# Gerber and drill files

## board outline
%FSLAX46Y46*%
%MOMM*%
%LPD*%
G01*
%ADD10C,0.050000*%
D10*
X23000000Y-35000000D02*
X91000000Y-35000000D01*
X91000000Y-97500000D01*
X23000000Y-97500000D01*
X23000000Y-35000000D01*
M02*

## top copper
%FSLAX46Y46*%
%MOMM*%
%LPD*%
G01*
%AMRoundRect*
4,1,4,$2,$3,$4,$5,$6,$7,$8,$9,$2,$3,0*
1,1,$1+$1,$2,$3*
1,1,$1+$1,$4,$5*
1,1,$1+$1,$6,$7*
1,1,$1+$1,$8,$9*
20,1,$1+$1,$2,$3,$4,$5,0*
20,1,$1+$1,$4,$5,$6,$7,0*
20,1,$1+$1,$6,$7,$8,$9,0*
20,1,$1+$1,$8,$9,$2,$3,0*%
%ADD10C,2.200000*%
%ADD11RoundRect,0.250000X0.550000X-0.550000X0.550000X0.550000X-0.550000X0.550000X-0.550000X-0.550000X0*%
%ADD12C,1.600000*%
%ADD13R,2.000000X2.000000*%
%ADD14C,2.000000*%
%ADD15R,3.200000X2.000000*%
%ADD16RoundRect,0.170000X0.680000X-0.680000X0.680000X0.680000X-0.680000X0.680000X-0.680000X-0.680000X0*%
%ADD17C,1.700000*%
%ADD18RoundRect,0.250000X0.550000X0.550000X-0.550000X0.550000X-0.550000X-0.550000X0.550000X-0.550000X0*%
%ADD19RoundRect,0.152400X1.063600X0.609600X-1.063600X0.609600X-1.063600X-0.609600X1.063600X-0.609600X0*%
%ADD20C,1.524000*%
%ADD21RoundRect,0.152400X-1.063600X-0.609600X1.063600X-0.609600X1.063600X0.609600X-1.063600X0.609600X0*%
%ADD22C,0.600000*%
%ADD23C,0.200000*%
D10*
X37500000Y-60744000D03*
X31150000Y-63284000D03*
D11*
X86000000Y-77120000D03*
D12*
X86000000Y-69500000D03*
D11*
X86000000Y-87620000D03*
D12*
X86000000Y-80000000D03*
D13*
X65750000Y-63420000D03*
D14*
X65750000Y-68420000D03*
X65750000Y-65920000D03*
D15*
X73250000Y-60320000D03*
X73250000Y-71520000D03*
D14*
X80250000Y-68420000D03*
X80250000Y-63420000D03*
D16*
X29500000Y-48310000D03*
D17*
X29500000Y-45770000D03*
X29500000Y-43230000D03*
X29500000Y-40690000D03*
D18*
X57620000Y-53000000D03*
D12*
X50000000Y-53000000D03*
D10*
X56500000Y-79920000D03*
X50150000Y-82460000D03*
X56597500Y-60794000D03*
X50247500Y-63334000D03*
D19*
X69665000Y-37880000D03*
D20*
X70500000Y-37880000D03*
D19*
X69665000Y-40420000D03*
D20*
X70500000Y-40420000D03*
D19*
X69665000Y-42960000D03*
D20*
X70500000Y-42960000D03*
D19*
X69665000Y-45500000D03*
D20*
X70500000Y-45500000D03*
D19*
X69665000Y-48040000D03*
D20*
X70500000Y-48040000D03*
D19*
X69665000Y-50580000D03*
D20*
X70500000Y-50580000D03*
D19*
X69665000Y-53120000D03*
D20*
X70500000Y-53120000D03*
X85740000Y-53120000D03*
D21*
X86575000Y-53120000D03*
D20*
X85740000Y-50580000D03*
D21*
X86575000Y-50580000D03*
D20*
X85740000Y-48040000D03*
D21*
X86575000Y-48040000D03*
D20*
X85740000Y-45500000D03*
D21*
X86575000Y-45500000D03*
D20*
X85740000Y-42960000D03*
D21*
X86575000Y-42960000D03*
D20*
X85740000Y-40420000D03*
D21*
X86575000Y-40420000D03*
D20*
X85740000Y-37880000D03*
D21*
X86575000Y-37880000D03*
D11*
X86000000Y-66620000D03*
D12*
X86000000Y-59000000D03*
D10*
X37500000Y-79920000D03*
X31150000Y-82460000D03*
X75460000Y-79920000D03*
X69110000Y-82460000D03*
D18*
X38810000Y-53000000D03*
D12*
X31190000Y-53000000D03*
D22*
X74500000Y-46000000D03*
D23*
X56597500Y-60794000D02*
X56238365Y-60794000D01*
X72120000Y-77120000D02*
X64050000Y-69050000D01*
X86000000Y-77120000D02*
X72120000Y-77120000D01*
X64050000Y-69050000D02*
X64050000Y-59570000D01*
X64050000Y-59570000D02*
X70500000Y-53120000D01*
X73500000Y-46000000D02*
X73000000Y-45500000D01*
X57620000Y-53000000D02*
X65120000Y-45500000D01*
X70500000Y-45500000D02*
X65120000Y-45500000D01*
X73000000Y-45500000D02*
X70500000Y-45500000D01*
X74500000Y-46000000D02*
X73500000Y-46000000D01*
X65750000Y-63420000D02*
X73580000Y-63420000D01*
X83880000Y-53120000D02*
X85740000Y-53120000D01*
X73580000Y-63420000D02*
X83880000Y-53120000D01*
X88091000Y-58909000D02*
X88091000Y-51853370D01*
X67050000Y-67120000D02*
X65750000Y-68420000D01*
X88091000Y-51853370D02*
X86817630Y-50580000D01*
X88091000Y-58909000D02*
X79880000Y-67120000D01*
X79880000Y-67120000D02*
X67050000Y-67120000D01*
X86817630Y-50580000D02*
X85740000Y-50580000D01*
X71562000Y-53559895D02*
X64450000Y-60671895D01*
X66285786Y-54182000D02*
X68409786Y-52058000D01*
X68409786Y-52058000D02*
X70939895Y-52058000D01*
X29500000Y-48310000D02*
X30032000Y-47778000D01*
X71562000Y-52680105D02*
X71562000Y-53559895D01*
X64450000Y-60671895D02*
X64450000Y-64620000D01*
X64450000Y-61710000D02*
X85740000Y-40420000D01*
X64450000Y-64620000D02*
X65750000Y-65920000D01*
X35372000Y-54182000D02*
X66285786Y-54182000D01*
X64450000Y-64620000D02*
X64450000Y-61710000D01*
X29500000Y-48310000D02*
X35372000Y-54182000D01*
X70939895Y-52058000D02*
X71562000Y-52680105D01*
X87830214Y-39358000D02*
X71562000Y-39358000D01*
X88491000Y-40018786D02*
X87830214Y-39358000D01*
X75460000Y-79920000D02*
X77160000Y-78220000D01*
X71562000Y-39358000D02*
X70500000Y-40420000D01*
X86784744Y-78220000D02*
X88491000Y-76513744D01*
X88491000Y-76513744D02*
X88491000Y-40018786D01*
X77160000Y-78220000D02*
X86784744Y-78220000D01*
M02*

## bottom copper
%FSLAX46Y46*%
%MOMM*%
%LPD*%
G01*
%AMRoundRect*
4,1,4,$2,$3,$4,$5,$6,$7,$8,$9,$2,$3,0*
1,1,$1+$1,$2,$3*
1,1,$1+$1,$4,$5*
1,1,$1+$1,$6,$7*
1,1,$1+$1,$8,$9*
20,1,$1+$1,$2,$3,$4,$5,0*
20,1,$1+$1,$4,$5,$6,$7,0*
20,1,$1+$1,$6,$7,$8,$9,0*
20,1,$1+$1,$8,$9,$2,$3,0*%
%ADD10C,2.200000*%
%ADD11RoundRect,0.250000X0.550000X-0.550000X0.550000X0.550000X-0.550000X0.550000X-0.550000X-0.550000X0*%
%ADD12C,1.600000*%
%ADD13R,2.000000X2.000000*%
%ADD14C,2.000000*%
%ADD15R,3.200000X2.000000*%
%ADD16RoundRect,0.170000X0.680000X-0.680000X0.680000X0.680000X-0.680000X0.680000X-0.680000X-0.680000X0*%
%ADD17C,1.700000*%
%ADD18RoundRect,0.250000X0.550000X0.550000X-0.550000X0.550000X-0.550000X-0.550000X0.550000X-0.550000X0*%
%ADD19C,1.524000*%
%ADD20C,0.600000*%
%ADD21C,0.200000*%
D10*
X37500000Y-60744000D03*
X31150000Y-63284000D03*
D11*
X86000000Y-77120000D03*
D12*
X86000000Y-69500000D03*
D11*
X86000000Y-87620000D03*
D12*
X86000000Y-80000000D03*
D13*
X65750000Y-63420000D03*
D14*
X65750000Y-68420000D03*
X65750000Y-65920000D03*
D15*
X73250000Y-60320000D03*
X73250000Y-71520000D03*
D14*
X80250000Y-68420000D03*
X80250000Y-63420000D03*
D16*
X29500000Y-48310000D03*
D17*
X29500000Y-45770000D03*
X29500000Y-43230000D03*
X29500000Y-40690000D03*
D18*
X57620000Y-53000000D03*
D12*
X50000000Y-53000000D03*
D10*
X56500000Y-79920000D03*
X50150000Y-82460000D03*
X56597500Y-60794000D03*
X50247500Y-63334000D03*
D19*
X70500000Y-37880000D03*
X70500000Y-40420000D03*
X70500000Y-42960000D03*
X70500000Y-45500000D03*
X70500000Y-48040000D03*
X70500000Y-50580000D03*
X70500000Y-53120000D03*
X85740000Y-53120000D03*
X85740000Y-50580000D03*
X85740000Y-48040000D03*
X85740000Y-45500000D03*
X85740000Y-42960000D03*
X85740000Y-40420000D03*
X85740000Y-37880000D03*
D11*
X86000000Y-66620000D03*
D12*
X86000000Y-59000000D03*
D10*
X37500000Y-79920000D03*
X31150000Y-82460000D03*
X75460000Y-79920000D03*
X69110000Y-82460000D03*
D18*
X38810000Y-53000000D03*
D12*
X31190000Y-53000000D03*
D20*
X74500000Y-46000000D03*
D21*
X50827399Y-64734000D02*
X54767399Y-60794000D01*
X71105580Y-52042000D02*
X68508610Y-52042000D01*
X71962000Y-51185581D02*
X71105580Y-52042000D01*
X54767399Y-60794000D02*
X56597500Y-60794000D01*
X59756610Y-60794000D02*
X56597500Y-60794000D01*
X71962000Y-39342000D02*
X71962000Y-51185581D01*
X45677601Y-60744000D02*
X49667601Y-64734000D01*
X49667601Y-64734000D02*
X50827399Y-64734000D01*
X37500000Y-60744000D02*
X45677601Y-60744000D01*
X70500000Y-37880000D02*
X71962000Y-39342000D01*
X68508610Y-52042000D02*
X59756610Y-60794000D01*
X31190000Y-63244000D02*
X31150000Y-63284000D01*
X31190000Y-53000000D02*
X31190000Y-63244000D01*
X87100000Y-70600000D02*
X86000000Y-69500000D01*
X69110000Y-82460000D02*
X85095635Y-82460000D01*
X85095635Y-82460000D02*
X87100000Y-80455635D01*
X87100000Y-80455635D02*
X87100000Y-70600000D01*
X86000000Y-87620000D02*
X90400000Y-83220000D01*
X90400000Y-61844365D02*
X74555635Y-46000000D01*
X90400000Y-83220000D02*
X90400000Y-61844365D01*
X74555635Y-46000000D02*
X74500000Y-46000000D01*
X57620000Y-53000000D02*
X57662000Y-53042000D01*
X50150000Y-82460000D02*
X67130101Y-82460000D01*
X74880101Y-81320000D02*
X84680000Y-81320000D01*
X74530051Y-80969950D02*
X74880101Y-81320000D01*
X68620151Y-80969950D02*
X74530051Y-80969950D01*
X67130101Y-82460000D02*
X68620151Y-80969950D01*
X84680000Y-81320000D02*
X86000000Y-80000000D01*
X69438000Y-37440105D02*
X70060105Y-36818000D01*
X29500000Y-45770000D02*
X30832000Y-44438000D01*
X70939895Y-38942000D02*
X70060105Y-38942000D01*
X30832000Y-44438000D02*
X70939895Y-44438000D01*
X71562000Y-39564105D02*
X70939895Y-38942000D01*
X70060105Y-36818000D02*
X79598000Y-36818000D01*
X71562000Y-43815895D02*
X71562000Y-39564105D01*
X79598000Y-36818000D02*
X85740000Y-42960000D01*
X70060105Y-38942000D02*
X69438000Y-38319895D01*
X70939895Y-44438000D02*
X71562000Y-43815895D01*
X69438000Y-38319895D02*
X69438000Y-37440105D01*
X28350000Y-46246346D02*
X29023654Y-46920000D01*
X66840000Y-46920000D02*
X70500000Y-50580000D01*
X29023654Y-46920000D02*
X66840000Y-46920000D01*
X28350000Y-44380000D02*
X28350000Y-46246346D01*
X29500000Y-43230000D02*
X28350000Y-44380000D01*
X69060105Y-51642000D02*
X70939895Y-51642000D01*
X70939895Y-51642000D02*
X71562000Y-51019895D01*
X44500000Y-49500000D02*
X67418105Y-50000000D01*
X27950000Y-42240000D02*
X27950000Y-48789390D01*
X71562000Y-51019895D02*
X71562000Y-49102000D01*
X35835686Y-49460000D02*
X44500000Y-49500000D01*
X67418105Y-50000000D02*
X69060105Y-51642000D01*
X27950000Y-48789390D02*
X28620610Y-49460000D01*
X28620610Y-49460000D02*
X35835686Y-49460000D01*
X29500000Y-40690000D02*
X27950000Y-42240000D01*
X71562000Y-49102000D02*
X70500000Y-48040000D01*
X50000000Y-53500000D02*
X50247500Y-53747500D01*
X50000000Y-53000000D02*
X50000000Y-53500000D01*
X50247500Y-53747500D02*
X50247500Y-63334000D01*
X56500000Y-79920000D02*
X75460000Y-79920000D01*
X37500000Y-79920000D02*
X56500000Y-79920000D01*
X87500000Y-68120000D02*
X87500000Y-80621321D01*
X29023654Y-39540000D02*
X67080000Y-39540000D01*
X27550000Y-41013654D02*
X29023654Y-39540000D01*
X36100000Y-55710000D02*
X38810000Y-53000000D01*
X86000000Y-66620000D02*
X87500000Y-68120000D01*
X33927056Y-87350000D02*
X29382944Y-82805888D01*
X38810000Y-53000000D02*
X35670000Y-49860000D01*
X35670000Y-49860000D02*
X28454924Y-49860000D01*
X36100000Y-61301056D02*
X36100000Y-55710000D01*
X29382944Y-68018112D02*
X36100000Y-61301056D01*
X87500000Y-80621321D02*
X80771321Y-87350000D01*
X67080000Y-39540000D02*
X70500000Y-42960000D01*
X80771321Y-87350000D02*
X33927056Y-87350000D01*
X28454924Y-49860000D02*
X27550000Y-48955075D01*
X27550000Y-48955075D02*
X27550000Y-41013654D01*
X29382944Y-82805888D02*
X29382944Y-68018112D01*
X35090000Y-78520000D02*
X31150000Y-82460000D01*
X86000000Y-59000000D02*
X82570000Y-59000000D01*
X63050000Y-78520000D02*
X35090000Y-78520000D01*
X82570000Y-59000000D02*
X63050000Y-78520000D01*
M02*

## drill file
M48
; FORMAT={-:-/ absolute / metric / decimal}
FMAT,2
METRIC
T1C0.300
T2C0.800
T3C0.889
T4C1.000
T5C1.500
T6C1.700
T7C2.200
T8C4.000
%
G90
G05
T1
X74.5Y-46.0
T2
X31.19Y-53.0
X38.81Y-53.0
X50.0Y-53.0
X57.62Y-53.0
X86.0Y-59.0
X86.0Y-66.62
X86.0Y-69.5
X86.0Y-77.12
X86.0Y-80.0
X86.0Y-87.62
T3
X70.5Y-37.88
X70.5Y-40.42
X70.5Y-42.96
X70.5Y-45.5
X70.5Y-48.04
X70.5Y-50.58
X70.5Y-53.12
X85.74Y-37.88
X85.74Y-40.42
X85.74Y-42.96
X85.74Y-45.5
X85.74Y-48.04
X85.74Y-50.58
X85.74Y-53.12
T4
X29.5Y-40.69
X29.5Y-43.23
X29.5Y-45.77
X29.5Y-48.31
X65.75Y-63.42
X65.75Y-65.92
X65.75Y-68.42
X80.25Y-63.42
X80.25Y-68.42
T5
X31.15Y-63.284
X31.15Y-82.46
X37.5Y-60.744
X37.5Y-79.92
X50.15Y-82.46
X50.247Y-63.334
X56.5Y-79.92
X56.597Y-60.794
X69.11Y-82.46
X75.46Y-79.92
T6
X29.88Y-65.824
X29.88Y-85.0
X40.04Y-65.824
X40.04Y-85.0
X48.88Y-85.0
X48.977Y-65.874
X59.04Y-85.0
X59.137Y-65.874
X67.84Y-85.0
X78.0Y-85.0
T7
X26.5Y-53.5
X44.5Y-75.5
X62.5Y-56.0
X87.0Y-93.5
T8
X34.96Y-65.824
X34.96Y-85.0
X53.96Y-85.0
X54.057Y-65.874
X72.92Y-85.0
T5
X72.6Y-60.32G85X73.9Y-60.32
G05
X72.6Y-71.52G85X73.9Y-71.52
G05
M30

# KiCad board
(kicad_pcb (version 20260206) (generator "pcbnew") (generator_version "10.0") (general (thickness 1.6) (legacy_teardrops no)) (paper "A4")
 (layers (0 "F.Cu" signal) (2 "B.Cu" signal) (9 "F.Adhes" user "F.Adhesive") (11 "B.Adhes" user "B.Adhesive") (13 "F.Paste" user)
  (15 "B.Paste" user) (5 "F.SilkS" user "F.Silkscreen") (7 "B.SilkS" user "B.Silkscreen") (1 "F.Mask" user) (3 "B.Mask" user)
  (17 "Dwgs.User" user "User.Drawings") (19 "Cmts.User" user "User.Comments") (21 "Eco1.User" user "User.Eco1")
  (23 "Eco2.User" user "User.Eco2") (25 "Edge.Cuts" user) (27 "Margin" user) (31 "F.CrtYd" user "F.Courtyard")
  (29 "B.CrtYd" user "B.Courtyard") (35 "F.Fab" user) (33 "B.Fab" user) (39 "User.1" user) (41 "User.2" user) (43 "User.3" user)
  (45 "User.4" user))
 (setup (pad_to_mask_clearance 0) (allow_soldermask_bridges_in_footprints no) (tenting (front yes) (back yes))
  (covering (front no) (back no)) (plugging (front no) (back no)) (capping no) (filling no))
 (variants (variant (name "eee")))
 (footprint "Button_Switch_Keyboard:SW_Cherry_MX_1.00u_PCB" (layer "F.Cu") (at 37.5 60.744)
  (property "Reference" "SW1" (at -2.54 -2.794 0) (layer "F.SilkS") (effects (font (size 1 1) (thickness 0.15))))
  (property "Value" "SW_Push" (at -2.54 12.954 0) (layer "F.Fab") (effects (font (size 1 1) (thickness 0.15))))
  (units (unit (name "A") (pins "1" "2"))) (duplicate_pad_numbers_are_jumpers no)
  (pad "" np_thru_hole circle (at -7.62 5.08) (size 1.7 1.7) (drill 1.7) (layers "*.Cu" "*.Mask"))
  (pad "" np_thru_hole circle (at -2.54 5.08) (size 4 4) (drill 4) (layers "*.Cu" "*.Mask"))
  (pad "" np_thru_hole circle (at 2.54 5.08) (size 1.7 1.7) (drill 1.7) (layers "*.Cu" "*.Mask"))
  (pad "1" thru_hole circle (at 0 0) (size 2.2 2.2) (drill 1.5) (layers "*.Cu" "*.Mask") (remove_unused_layers no) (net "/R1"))
  (pad "2" thru_hole circle (at -6.35 2.54) (size 2.2 2.2) (drill 1.5) (layers "*.Cu" "*.Mask") (remove_unused_layers no) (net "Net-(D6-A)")))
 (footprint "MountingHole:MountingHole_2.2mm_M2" (layer "F.Cu") (at 87 93.5)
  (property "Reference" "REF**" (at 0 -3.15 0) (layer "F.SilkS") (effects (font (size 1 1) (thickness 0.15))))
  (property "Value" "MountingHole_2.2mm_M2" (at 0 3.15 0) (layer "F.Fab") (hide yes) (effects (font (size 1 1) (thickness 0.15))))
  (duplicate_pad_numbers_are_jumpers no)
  (pad "" np_thru_hole circle (at 0 0) (size 2.2 2.2) (drill 2.2) (layers "*.Cu" "*.Mask")))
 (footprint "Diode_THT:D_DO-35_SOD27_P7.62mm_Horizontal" (layer "F.Cu") (at 86 77.12 90)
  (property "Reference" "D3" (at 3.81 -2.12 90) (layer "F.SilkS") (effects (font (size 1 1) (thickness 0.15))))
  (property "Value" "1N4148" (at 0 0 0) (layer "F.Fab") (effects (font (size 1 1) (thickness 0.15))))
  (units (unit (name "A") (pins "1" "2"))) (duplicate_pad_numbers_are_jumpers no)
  (pad "1" thru_hole roundrect (at 0 0 90) (size 1.6 1.6) (drill 0.8) (layers "*.Cu" "*.Mask") (remove_unused_layers no)
   (roundrect_rratio 0.15625) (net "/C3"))
  (pad "2" thru_hole circle (at 7.62 0 90) (size 1.6 1.6) (drill 0.8) (layers "*.Cu" "*.Mask") (remove_unused_layers no) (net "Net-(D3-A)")))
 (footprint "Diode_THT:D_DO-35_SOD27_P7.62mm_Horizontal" (layer "F.Cu") (at 86 87.62 90)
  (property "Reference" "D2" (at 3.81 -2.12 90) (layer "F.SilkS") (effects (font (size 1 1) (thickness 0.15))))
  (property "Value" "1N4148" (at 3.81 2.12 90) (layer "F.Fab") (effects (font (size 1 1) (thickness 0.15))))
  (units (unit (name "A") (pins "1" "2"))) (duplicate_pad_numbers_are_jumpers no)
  (pad "1" thru_hole roundrect (at 0 0 90) (size 1.6 1.6) (drill 0.8) (layers "*.Cu" "*.Mask") (remove_unused_layers no)
   (roundrect_rratio 0.15625) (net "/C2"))
  (pad "2" thru_hole circle (at 7.62 0 90) (size 1.6 1.6) (drill 0.8) (layers "*.Cu" "*.Mask") (remove_unused_layers no) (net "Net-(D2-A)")))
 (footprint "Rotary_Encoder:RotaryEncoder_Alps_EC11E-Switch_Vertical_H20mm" (layer "F.Cu") (at 65.75 63.42)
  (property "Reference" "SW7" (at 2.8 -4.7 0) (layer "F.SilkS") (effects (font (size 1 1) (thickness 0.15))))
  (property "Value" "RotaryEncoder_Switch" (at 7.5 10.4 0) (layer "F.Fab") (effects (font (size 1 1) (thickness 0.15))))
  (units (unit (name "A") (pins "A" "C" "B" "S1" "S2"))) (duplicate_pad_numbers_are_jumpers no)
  (pad "A" thru_hole rect (at 0 0) (size 2 2) (drill 1) (layers "*.Cu" "*.Mask") (remove_unused_layers no) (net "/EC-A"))
  (pad "B" thru_hole circle (at 0 5) (size 2 2) (drill 1) (layers "*.Cu" "*.Mask") (remove_unused_layers no) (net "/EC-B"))
  (pad "C" thru_hole circle (at 0 2.5) (size 2 2) (drill 1) (layers "*.Cu" "*.Mask") (remove_unused_layers no) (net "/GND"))
  (pad "MP" thru_hole rect (at 7.5 -3.1) (size 3.2 2) (drill oval 2.8 1.5) (layers "*.Cu" "*.Mask") (remove_unused_layers no))
  (pad "MP" thru_hole rect (at 7.5 8.1) (size 3.2 2) (drill oval 2.8 1.5) (layers "*.Cu" "*.Mask") (remove_unused_layers no))
  (pad "S1" thru_hole circle (at 14.5 5) (size 2 2) (drill 1) (layers "*.Cu" "*.Mask") (remove_unused_layers no)
   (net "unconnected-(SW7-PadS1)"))
  (pad "S2" thru_hole circle (at 14.5 0) (size 2 2) (drill 1) (layers "*.Cu" "*.Mask") (remove_unused_layers no)
   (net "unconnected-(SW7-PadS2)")))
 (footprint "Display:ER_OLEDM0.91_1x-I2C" (layer "F.Cu") (at 29.5 48.31 90)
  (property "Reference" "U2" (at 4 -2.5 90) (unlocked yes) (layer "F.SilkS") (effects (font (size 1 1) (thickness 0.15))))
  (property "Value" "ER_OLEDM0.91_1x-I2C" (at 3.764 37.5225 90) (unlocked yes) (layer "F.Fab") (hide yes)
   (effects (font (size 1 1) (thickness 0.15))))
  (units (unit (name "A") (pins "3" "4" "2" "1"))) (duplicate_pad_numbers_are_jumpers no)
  (pad "1" thru_hole roundrect (at 0 0 90) (size 1.7 1.7) (drill 1) (layers "*.Cu" "*.Mask") (remove_unused_layers no)
   (roundrect_rratio 0.1) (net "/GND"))
  (pad "2" thru_hole circle (at 2.54 0 90) (size 1.7 1.7) (drill 1) (layers "*.Cu" "*.Mask") (remove_unused_layers no) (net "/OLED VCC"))
  (pad "3" thru_hole circle (at 5.08 0 90) (size 1.7 1.7) (drill 1) (layers "*.Cu" "*.Mask") (remove_unused_layers no) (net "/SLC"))
  (pad "4" thru_hole circle (at 7.62 0 90) (size 1.7 1.7) (drill 1) (layers "*.Cu" "*.Mask") (remove_unused_layers no) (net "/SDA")))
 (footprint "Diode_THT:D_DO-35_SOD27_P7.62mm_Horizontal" (layer "F.Cu") (at 57.62 53 180)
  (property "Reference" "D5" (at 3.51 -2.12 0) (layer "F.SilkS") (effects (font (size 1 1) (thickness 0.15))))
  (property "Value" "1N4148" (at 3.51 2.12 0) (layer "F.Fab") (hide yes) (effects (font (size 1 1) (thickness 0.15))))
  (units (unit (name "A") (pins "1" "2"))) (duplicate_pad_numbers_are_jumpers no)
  (pad "1" thru_hole roundrect (at 0 0 180) (size 1.6 1.6) (drill 0.8) (layers "*.Cu" "*.Mask") (remove_unused_layers no)
   (roundrect_rratio 0.15625) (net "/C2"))
  (pad "2" thru_hole circle (at 7.62 0 180) (size 1.6 1.6) (drill 0.8) (layers "*.Cu" "*.Mask") (remove_unused_layers no) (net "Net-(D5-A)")))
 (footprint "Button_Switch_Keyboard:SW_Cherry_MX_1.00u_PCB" (layer "F.Cu") (at 56.5 79.92)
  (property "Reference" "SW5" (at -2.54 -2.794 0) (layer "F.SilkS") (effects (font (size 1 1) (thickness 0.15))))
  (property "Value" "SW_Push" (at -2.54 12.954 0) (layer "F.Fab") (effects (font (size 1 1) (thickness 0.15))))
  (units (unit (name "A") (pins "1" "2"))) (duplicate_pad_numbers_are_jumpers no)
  (pad "" np_thru_hole circle (at -7.62 5.08) (size 1.7 1.7) (drill 1.7) (layers "*.Cu" "*.Mask"))
  (pad "" np_thru_hole circle (at -2.54 5.08) (size 4 4) (drill 4) (layers "*.Cu" "*.Mask"))
  (pad "" np_thru_hole circle (at 2.54 5.08) (size 1.7 1.7) (drill 1.7) (layers "*.Cu" "*.Mask"))
  (pad "1" thru_hole circle (at 0 0) (size 2.2 2.2) (drill 1.5) (layers "*.Cu" "*.Mask") (remove_unused_layers no) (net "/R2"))
  (pad "2" thru_hole circle (at -6.35 2.54) (size 2.2 2.2) (drill 1.5) (layers "*.Cu" "*.Mask") (remove_unused_layers no) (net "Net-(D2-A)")))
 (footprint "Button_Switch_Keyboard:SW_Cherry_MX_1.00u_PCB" (layer "F.Cu") (at 56.5975 60.794)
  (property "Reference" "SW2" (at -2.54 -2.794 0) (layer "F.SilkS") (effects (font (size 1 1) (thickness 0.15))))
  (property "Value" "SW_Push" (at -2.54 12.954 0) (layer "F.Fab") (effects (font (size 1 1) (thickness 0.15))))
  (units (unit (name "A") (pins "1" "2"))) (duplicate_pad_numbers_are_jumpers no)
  (pad "" np_thru_hole circle (at -7.62 5.08) (size 1.7 1.7) (drill 1.7) (layers "*.Cu" "*.Mask"))
  (pad "" np_thru_hole circle (at -2.54 5.08) (size 4 4) (drill 4) (layers "*.Cu" "*.Mask"))
  (pad "" np_thru_hole circle (at 2.54 5.08) (size 1.7 1.7) (drill 1.7) (layers "*.Cu" "*.Mask"))
  (pad "1" thru_hole circle (at 0 0) (size 2.2 2.2) (drill 1.5) (layers "*.Cu" "*.Mask") (remove_unused_layers no) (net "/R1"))
  (pad "2" thru_hole circle (at -6.35 2.54) (size 2.2 2.2) (drill 1.5) (layers "*.Cu" "*.Mask") (remove_unused_layers no) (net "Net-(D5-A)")))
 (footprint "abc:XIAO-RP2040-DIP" (layer "F.Cu") (at 78.12 45.5 90)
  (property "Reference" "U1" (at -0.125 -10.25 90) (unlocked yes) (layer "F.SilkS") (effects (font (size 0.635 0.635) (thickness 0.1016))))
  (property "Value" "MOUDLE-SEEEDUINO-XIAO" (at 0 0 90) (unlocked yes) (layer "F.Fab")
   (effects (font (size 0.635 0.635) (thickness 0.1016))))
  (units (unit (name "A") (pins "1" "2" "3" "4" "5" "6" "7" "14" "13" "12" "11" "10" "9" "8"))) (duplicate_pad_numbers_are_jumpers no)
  (pad "1" smd roundrect (at 7.62 -8.455 180) (size 2.432 1.524) (layers "F.Cu" "F.Mask") (roundrect_rratio 0.1) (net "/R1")
   (thermal_bridge_angle 45))
  (pad "1" thru_hole circle (at 7.62 -7.62 180) (size 1.524 1.524) (drill 0.889) (layers "*.Cu" "*.Mask") (remove_unused_layers no)
   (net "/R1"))
  (pad "2" smd roundrect (at 5.08 -8.455 180) (size 2.432 1.524) (layers "F.Cu" "F.Mask") (roundrect_rratio 0.1) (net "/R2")
   (thermal_bridge_angle 45))
  (pad "2" thru_hole circle (at 5.08 -7.62 180) (size 1.524 1.524) (drill 0.889) (layers "*.Cu" "*.Mask") (remove_unused_layers no)
   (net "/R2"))
  (pad "3" smd roundrect (at 2.54 -8.455 180) (size 2.432 1.524) (layers "F.Cu" "F.Mask") (roundrect_rratio 0.1) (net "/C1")
   (thermal_bridge_angle 45))
  (pad "3" thru_hole circle (at 2.54 -7.62 180) (size 1.524 1.524) (drill 0.889) (layers "*.Cu" "*.Mask") (remove_unused_layers no)
   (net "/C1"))
  (pad "4" smd roundrect (at 0 -8.455 180) (size 2.432 1.524) (layers "F.Cu" "F.Mask") (roundrect_rratio 0.1) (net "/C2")
   (thermal_bridge_angle 45))
  (pad "4" thru_hole circle (at 0 -7.62 180) (size 1.524 1.524) (drill 0.889) (layers "*.Cu" "*.Mask") (remove_unused_layers no) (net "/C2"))
  (pad "5" smd roundrect (at -2.54 -8.455 180) (size 2.432 1.524) (layers "F.Cu" "F.Mask") (roundrect_rratio 0.1) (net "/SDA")
   (thermal_bridge_angle 45))
  (pad "5" thru_hole circle (at -2.54 -7.62 180) (size 1.524 1.524) (drill 0.889) (layers "*.Cu" "*.Mask") (remove_unused_layers no)
   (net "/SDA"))
  (pad "6" smd roundrect (at -5.08 -8.455 180) (size 2.432 1.524) (layers "F.Cu" "F.Mask") (roundrect_rratio 0.1) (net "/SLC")
   (thermal_bridge_angle 45))
  (pad "6" thru_hole circle (at -5.08 -7.62 180) (size 1.524 1.524) (drill 0.889) (layers "*.Cu" "*.Mask") (remove_unused_layers no)
   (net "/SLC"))
  (pad "7" smd roundrect (at -7.62 -8.455 180) (size 2.432 1.524) (layers "F.Cu" "F.Mask") (roundrect_rratio 0.1) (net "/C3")
   (thermal_bridge_angle 45))
  (pad "7" thru_hole circle (at -7.62 -7.62 180) (size 1.524 1.524) (drill 0.889) (layers "*.Cu" "*.Mask") (remove_unused_layers no)
   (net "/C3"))
  (pad "8" thru_hole circle (at -7.62 7.62) (size 1.524 1.524) (drill 0.889) (layers "*.Cu" "*.Mask") (remove_unused_layers no)
   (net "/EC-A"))
  (pad "8" smd roundrect (at -7.62 8.455) (size 2.432 1.524) (layers "F.Cu" "F.Mask") (roundrect_rratio 0.1) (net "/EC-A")
   (thermal_bridge_angle 45))
  (pad "9" thru_hole circle (at -5.08 7.62) (size 1.524 1.524) (drill 0.889) (layers "*.Cu" "*.Mask") (remove_unused_layers no)
   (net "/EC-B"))
  (pad "9" smd roundrect (at -5.08 8.455) (size 2.432 1.524) (layers "F.Cu" "F.Mask") (roundrect_rratio 0.1) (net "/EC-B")
   (thermal_bridge_angle 45))
  (pad "10" thru_hole circle (at -2.54 7.62) (size 1.524 1.524) (drill 0.889) (layers "*.Cu" "*.Mask") (remove_unused_layers no)
   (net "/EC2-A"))
  (pad "10" smd roundrect (at -2.54 8.455) (size 2.432 1.524) (layers "F.Cu" "F.Mask") (roundrect_rratio 0.1) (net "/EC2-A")
   (thermal_bridge_angle 45))
  (pad "11" thru_hole circle (at 0 7.62) (size 1.524 1.524) (drill 0.889) (layers "*.Cu" "*.Mask") (remove_unused_layers no) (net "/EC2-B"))
  (pad "11" smd roundrect (at 0 8.455) (size 2.432 1.524) (layers "F.Cu" "F.Mask") (roundrect_rratio 0.1) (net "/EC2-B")
   (thermal_bridge_angle 45))
  (pad "12" thru_hole circle (at 2.54 7.62) (size 1.524 1.524) (drill 0.889) (layers "*.Cu" "*.Mask") (remove_unused_layers no)
   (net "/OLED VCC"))
  (pad "12" smd roundrect (at 2.54 8.455) (size 2.432 1.524) (layers "F.Cu" "F.Mask") (roundrect_rratio 0.1) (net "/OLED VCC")
   (thermal_bridge_angle 45))
  (pad "13" thru_hole circle (at 5.08 7.62) (size 1.524 1.524) (drill 0.889) (layers "*.Cu" "*.Mask") (remove_unused_layers no) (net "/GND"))
  (pad "13" smd roundrect (at 5.08 8.455) (size 2.432 1.524) (layers "F.Cu" "F.Mask") (roundrect_rratio 0.1) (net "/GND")
   (thermal_bridge_angle 45))
  (pad "14" thru_hole circle (at 7.62 7.62) (size 1.524 1.524) (drill 0.889) (layers "*.Cu" "*.Mask") (remove_unused_layers no)
   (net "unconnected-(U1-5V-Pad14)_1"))
  (pad "14" smd roundrect (at 7.62 8.455) (size 2.432 1.524) (layers "F.Cu" "F.Mask") (roundrect_rratio 0.1)
   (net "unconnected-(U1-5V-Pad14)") (thermal_bridge_angle 45)))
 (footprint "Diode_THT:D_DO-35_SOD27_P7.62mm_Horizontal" (layer "F.Cu") (at 86 66.62 90)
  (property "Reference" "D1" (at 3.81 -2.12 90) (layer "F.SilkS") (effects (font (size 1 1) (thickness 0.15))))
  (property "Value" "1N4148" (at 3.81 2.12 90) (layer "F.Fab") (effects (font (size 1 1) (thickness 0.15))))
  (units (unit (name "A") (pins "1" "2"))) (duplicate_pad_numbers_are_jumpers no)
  (pad "1" thru_hole roundrect (at 0 0 90) (size 1.6 1.6) (drill 0.8) (layers "*.Cu" "*.Mask") (remove_unused_layers no)
   (roundrect_rratio 0.15625) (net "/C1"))
  (pad "2" thru_hole circle (at 7.62 0 90) (size 1.6 1.6) (drill 0.8) (layers "*.Cu" "*.Mask") (remove_unused_layers no) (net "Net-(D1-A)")))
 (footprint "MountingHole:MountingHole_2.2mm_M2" (layer "F.Cu") (at 26.5 53.5)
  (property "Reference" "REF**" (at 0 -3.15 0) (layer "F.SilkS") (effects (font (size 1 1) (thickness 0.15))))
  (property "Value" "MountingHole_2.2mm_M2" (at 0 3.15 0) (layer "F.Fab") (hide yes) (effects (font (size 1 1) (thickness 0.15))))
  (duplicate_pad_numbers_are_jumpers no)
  (pad "" np_thru_hole circle (at 0 0) (size 2.2 2.2) (drill 2.2) (layers "*.Cu" "*.Mask")))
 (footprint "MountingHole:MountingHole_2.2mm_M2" (layer "F.Cu") (at 62.5 56)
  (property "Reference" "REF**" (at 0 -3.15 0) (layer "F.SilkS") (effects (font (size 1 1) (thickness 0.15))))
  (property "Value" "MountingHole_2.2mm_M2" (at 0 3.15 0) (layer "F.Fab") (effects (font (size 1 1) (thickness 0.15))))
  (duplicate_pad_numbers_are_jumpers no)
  (pad "" np_thru_hole circle (at 0 0) (size 2.2 2.2) (drill 2.2) (layers "*.Cu" "*.Mask")))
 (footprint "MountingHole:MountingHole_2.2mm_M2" (layer "F.Cu") (at 44.5 75.5)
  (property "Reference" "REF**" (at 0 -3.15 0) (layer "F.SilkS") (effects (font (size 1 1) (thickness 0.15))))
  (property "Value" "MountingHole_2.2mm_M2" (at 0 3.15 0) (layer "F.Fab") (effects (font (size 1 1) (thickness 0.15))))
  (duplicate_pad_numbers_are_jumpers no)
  (pad "" np_thru_hole circle (at 0 0) (size 2.2 2.2) (drill 2.2) (layers "*.Cu" "*.Mask")))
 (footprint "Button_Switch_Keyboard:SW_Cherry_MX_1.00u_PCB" (layer "F.Cu") (at 37.5 79.92)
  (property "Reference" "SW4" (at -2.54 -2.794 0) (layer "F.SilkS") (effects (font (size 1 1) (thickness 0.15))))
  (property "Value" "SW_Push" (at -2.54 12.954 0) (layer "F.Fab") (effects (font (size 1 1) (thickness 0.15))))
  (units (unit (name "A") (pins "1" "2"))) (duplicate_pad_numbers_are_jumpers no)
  (pad "" np_thru_hole circle (at -7.62 5.08) (size 1.7 1.7) (drill 1.7) (layers "*.Cu" "*.Mask"))
  (pad "" np_thru_hole circle (at -2.54 5.08) (size 4 4) (drill 4) (layers "*.Cu" "*.Mask"))
  (pad "" np_thru_hole circle (at 2.54 5.08) (size 1.7 1.7) (drill 1.7) (layers "*.Cu" "*.Mask"))
  (pad "1" thru_hole circle (at 0 0) (size 2.2 2.2) (drill 1.5) (layers "*.Cu" "*.Mask") (remove_unused_layers no) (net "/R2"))
  (pad "2" thru_hole circle (at -6.35 2.54) (size 2.2 2.2) (drill 1.5) (layers "*.Cu" "*.Mask") (remove_unused_layers no) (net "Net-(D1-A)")))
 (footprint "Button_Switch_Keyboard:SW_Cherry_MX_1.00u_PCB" (layer "F.Cu") (at 75.46 79.92)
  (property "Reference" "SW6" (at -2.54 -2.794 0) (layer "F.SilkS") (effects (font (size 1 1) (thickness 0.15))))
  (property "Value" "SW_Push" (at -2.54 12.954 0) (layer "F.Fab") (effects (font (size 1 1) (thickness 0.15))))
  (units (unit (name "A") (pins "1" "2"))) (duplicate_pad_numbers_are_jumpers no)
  (pad "" np_thru_hole circle (at -7.62 5.08) (size 1.7 1.7) (drill 1.7) (layers "*.Cu" "*.Mask"))
  (pad "" np_thru_hole circle (at -2.54 5.08) (size 4 4) (drill 4) (layers "*.Cu" "*.Mask"))
  (pad "" np_thru_hole circle (at 2.54 5.08) (size 1.7 1.7) (drill 1.7) (layers "*.Cu" "*.Mask"))
  (pad "1" thru_hole circle (at 0 0) (size 2.2 2.2) (drill 1.5) (layers "*.Cu" "*.Mask") (remove_unused_layers no) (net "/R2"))
  (pad "2" thru_hole circle (at -6.35 2.54) (size 2.2 2.2) (drill 1.5) (layers "*.Cu" "*.Mask") (remove_unused_layers no) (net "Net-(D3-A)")))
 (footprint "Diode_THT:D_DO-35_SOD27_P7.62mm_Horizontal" (layer "F.Cu") (at 38.81 53 180)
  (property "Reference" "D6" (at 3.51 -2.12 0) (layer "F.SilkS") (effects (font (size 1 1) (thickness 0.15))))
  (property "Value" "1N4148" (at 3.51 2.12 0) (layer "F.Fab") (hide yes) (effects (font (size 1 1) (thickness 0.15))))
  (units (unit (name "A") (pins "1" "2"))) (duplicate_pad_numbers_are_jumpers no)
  (pad "1" thru_hole roundrect (at 0 0 180) (size 1.6 1.6) (drill 0.8) (layers "*.Cu" "*.Mask") (remove_unused_layers no)
   (roundrect_rratio 0.15625) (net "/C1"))
  (pad "2" thru_hole circle (at 7.62 0 180) (size 1.6 1.6) (drill 0.8) (layers "*.Cu" "*.Mask") (remove_unused_layers no) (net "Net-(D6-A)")))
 (gr_rect (start 23 35) (end 91 97.5) (stroke (width 0.05) (type default)) (fill no) (layer "Edge.Cuts"))
 (segment (start 56.5975 60.794) (end 56.238365 60.794) (width 0.2) (layer "F.Cu") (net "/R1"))
 (segment (start 50.827399 64.734) (end 54.767399 60.794) (width 0.2) (layer "B.Cu") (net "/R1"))
 (segment (start 71.10558 52.042) (end 68.50861 52.042) (width 0.2) (layer "B.Cu") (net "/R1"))
 (segment (start 71.962 51.185581) (end 71.10558 52.042) (width 0.2) (layer "B.Cu") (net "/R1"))
 (segment (start 54.767399 60.794) (end 56.5975 60.794) (width 0.2) (layer "B.Cu") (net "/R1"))
 (segment (start 59.75661 60.794) (end 56.5975 60.794) (width 0.2) (layer "B.Cu") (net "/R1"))
 (segment (start 71.962 39.342) (end 71.962 51.185581) (width 0.2) (layer "B.Cu") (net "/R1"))
 (segment (start 45.677601 60.744) (end 49.667601 64.734) (width 0.2) (layer "B.Cu") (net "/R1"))
 (segment (start 49.667601 64.734) (end 50.827399 64.734) (width 0.2) (layer "B.Cu") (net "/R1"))
 (segment (start 37.5 60.744) (end 45.677601 60.744) (width 0.2) (layer "B.Cu") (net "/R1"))
 (segment (start 70.5 37.88) (end 71.962 39.342) (width 0.2) (layer "B.Cu") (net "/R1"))
 (segment (start 68.50861 52.042) (end 59.75661 60.794) (width 0.2) (layer "B.Cu") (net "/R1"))
 (segment (start 31.19 63.244) (end 31.15 63.284) (width 0.2) (layer "B.Cu") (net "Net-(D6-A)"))
 (segment (start 31.19 53) (end 31.19 63.244) (width 0.2) (layer "B.Cu") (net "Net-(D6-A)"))
 (segment (start 72.12 77.12) (end 64.05 69.05) (width 0.2) (layer "F.Cu") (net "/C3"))
 (segment (start 86 77.12) (end 72.12 77.12) (width 0.2) (layer "F.Cu") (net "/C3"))
 (segment (start 64.05 69.05) (end 64.05 59.57) (width 0.2) (layer "F.Cu") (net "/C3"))
 (segment (start 64.05 59.57) (end 70.5 53.12) (width 0.2) (layer "F.Cu") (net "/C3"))
 (segment (start 87.1 70.6) (end 86 69.5) (width 0.2) (layer "B.Cu") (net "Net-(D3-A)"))
 (segment (start 69.11 82.46) (end 85.095635 82.46) (width 0.2) (layer "B.Cu") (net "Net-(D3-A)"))
 (segment (start 85.095635 82.46) (end 87.1 80.455635) (width 0.2) (layer "B.Cu") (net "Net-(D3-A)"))
 (segment (start 87.1 80.455635) (end 87.1 70.6) (width 0.2) (layer "B.Cu") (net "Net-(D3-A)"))
 (segment (start 73.5 46) (end 73 45.5) (width 0.2) (layer "F.Cu") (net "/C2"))
 (segment (start 57.62 53) (end 65.12 45.5) (width 0.2) (layer "F.Cu") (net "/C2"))
 (segment (start 70.5 45.5) (end 65.12 45.5) (width 0.2) (layer "F.Cu") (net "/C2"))
 (segment (start 73 45.5) (end 70.5 45.5) (width 0.2) (layer "F.Cu") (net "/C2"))
 (segment (start 74.5 46) (end 73.5 46) (width 0.2) (layer "F.Cu") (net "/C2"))
 (via (at 74.5 46) (size 0.6) (drill 0.3) (layers "F.Cu" "B.Cu") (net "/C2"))
 (segment (start 86 87.62) (end 90.4 83.22) (width 0.2) (layer "B.Cu") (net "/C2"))
 (segment (start 90.4 61.844365) (end 74.555635 46) (width 0.2) (layer "B.Cu") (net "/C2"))
 (segment (start 90.4 83.22) (end 90.4 61.844365) (width 0.2) (layer "B.Cu") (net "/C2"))
 (segment (start 74.555635 46) (end 74.5 46) (width 0.2) (layer "B.Cu") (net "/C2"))
 (segment (start 57.62 53) (end 57.662 53.042) (width 0.2) (layer "B.Cu") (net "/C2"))
 (segment (start 50.15 82.46) (end 67.130101 82.46) (width 0.2) (layer "B.Cu") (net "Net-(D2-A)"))
 (segment (start 74.880101 81.32) (end 84.68 81.32) (width 0.2) (layer "B.Cu") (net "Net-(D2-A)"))
 (segment (start 74.530051 80.96995) (end 74.880101 81.32) (width 0.2) (layer "B.Cu") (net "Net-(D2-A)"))
 (segment (start 68.620151 80.96995) (end 74.530051 80.96995) (width 0.2) (layer "B.Cu") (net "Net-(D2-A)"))
 (segment (start 67.130101 82.46) (end 68.620151 80.96995) (width 0.2) (layer "B.Cu") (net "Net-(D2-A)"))
 (segment (start 84.68 81.32) (end 86 80) (width 0.2) (layer "B.Cu") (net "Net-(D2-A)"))
 (segment (start 65.75 63.42) (end 73.58 63.42) (width 0.2) (layer "F.Cu") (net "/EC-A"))
 (segment (start 83.88 53.12) (end 85.74 53.12) (width 0.2) (layer "F.Cu") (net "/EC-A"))
 (segment (start 73.58 63.42) (end 83.88 53.12) (width 0.2) (layer "F.Cu") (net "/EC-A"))
 (segment (start 88.091 58.909) (end 88.091 51.85337) (width 0.2) (layer "F.Cu") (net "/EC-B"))
 (segment (start 67.05 67.12) (end 65.75 68.42) (width 0.2) (layer "F.Cu") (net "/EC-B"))
 (segment (start 88.091 51.85337) (end 86.81763 50.58) (width 0.2) (layer "F.Cu") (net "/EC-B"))
 (segment (start 88.091 58.909) (end 79.88 67.12) (width 0.2) (layer "F.Cu") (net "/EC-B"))
 (segment (start 79.88 67.12) (end 67.05 67.12) (width 0.2) (layer "F.Cu") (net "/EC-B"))
 (segment (start 86.81763 50.58) (end 85.74 50.58) (width 0.2) (layer "F.Cu") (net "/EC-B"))
 (segment (start 71.562 53.559895) (end 64.45 60.671895) (width 0.2) (layer "F.Cu") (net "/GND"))
 (segment (start 66.285786 54.182) (end 68.409786 52.058) (width 0.2) (layer "F.Cu") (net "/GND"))
 (segment (start 68.409786 52.058) (end 70.939895 52.058) (width 0.2) (layer "F.Cu") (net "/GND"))
 (segment (start 29.5 48.31) (end 30.032 47.778) (width 0.2) (layer "F.Cu") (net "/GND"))
 (segment (start 71.562 52.680105) (end 71.562 53.559895) (width 0.2) (layer "F.Cu") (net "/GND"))
 (segment (start 64.45 60.671895) (end 64.45 64.62) (width 0.2) (layer "F.Cu") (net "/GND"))
 (segment (start 64.45 61.71) (end 85.74 40.42) (width 0.2) (layer "F.Cu") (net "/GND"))
 (segment (start 64.45 64.62) (end 65.75 65.92) (width 0.2) (layer "F.Cu") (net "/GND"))
 (segment (start 35.372 54.182) (end 66.285786 54.182) (width 0.2) (layer "F.Cu") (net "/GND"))
 (segment (start 64.45 64.62) (end 64.45 61.71) (width 0.2) (layer "F.Cu") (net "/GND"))
 (segment (start 29.5 48.31) (end 35.372 54.182) (width 0.2) (layer "F.Cu") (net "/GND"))
 (segment (start 70.939895 52.058) (end 71.562 52.680105) (width 0.2) (layer "F.Cu") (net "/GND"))
 (segment (start 69.438 37.440105) (end 70.060105 36.818) (width 0.2) (layer "B.Cu") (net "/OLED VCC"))
 (segment (start 29.5 45.77) (end 30.832 44.438) (width 0.2) (layer "B.Cu") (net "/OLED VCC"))
 (segment (start 70.939895 38.942) (end 70.060105 38.942) (width 0.2) (layer "B.Cu") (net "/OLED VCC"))
 (segment (start 30.832 44.438) (end 70.939895 44.438) (width 0.2) (layer "B.Cu") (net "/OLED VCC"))
 (segment (start 71.562 39.564105) (end 70.939895 38.942) (width 0.2) (layer "B.Cu") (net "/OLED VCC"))
 (segment (start 70.060105 36.818) (end 79.598 36.818) (width 0.2) (layer "B.Cu") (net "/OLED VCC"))
 (segment (start 71.562 43.815895) (end 71.562 39.564105) (width 0.2) (layer "B.Cu") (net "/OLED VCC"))
 (segment (start 79.598 36.818) (end 85.74 42.96) (width 0.2) (layer "B.Cu") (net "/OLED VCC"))
 (segment (start 70.060105 38.942) (end 69.438 38.319895) (width 0.2) (layer "B.Cu") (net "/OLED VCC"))
 (segment (start 70.939895 44.438) (end 71.562 43.815895) (width 0.2) (layer "B.Cu") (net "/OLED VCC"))
 (segment (start 69.438 38.319895) (end 69.438 37.440105) (width 0.2) (layer "B.Cu") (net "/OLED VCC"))
 (segment (start 28.35 46.246346) (end 29.023654 46.92) (width 0.2) (layer "B.Cu") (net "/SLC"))
 (segment (start 66.84 46.92) (end 70.5 50.58) (width 0.2) (layer "B.Cu") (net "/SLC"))
 (segment (start 29.023654 46.92) (end 66.84 46.92) (width 0.2) (layer "B.Cu") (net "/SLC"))
 (segment (start 28.35 44.38) (end 28.35 46.246346) (width 0.2) (layer "B.Cu") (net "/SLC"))
 (segment (start 29.5 43.23) (end 28.35 44.38) (width 0.2) (layer "B.Cu") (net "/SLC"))
 (segment (start 69.060105 51.642) (end 70.939895 51.642) (width 0.2) (layer "B.Cu") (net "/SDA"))
 (segment (start 70.939895 51.642) (end 71.562 51.019895) (width 0.2) (layer "B.Cu") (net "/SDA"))
 (segment (start 44.5 49.5) (end 67.418105 50) (width 0.2) (layer "B.Cu") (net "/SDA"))
 (segment (start 27.95 42.24) (end 27.95 48.78939) (width 0.2) (layer "B.Cu") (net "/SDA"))
 (segment (start 71.562 51.019895) (end 71.562 49.102) (width 0.2) (layer "B.Cu") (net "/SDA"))
 (segment (start 35.835686 49.46) (end 44.5 49.5) (width 0.2) (layer "B.Cu") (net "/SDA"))
 (segment (start 67.418105 50) (end 69.060105 51.642) (width 0.2) (layer "B.Cu") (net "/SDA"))
 (segment (start 27.95 48.78939) (end 28.62061 49.46) (width 0.2) (layer "B.Cu") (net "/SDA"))
 (segment (start 28.62061 49.46) (end 35.835686 49.46) (width 0.2) (layer "B.Cu") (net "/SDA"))
 (segment (start 29.5 40.69) (end 27.95 42.24) (width 0.2) (layer "B.Cu") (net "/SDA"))
 (segment (start 71.562 49.102) (end 70.5 48.04) (width 0.2) (layer "B.Cu") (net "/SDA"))
 (segment (start 50 53.5) (end 50.2475 53.7475) (width 0.2) (layer "B.Cu") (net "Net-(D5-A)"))
 (segment (start 50 53) (end 50 53.5) (width 0.2) (layer "B.Cu") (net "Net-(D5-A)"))
 (segment (start 50.2475 53.7475) (end 50.2475 63.334) (width 0.2) (layer "B.Cu") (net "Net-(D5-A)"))
 (segment (start 87.830214 39.358) (end 71.562 39.358) (width 0.2) (layer "F.Cu") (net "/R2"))
 (segment (start 88.491 40.018786) (end 87.830214 39.358) (width 0.2) (layer "F.Cu") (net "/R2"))
 (segment (start 75.46 79.92) (end 77.16 78.22) (width 0.2) (layer "F.Cu") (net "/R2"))
 (segment (start 71.562 39.358) (end 70.5 40.42) (width 0.2) (layer "F.Cu") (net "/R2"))
 (segment (start 86.784744 78.22) (end 88.491 76.513744) (width 0.2) (layer "F.Cu") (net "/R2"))
 (segment (start 88.491 76.513744) (end 88.491 40.018786) (width 0.2) (layer "F.Cu") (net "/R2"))
 (segment (start 77.16 78.22) (end 86.784744 78.22) (width 0.2) (layer "F.Cu") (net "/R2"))
 (segment (start 56.5 79.92) (end 75.46 79.92) (width 0.2) (layer "B.Cu") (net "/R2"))
 (segment (start 37.5 79.92) (end 56.5 79.92) (width 0.2) (layer "B.Cu") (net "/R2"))
 (segment (start 87.5 68.12) (end 87.5 80.621321) (width 0.2) (layer "B.Cu") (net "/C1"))
 (segment (start 29.023654 39.54) (end 67.08 39.54) (width 0.2) (layer "B.Cu") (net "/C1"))
 (segment (start 27.55 41.013654) (end 29.023654 39.54) (width 0.2) (layer "B.Cu") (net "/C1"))
 (segment (start 36.1 55.71) (end 38.81 53) (width 0.2) (layer "B.Cu") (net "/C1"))
 (segment (start 86 66.62) (end 87.5 68.12) (width 0.2) (layer "B.Cu") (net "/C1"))
 (segment (start 33.927056 87.35) (end 29.382944 82.805888) (width 0.2) (layer "B.Cu") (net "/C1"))
 (segment (start 38.81 53) (end 35.67 49.86) (width 0.2) (layer "B.Cu") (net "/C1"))
 (segment (start 35.67 49.86) (end 28.454924 49.86) (width 0.2) (layer "B.Cu") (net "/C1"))
 (segment (start 36.1 61.301056) (end 36.1 55.71) (width 0.2) (layer "B.Cu") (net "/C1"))
 (segment (start 29.382944 68.018112) (end 36.1 61.301056) (width 0.2) (layer "B.Cu") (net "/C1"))
 (segment (start 87.5 80.621321) (end 80.771321 87.35) (width 0.2) (layer "B.Cu") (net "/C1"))
 (segment (start 67.08 39.54) (end 70.5 42.96) (width 0.2) (layer "B.Cu") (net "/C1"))
 (segment (start 80.771321 87.35) (end 33.927056 87.35) (width 0.2) (layer "B.Cu") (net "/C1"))
 (segment (start 28.454924 49.86) (end 27.55 48.955075) (width 0.2) (layer "B.Cu") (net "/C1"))
 (segment (start 27.55 48.955075) (end 27.55 41.013654) (width 0.2) (layer "B.Cu") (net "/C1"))
 (segment (start 29.382944 82.805888) (end 29.382944 68.018112) (width 0.2) (layer "B.Cu") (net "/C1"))
 (segment (start 35.09 78.52) (end 31.15 82.46) (width 0.2) (layer "B.Cu") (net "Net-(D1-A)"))
 (segment (start 86 59) (end 82.57 59) (width 0.2) (layer "B.Cu") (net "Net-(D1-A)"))
 (segment (start 63.05 78.52) (end 35.09 78.52) (width 0.2) (layer "B.Cu") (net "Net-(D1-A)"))
 (segment (start 82.57 59) (end 63.05 78.52) (width 0.2) (layer "B.Cu") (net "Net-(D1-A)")))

